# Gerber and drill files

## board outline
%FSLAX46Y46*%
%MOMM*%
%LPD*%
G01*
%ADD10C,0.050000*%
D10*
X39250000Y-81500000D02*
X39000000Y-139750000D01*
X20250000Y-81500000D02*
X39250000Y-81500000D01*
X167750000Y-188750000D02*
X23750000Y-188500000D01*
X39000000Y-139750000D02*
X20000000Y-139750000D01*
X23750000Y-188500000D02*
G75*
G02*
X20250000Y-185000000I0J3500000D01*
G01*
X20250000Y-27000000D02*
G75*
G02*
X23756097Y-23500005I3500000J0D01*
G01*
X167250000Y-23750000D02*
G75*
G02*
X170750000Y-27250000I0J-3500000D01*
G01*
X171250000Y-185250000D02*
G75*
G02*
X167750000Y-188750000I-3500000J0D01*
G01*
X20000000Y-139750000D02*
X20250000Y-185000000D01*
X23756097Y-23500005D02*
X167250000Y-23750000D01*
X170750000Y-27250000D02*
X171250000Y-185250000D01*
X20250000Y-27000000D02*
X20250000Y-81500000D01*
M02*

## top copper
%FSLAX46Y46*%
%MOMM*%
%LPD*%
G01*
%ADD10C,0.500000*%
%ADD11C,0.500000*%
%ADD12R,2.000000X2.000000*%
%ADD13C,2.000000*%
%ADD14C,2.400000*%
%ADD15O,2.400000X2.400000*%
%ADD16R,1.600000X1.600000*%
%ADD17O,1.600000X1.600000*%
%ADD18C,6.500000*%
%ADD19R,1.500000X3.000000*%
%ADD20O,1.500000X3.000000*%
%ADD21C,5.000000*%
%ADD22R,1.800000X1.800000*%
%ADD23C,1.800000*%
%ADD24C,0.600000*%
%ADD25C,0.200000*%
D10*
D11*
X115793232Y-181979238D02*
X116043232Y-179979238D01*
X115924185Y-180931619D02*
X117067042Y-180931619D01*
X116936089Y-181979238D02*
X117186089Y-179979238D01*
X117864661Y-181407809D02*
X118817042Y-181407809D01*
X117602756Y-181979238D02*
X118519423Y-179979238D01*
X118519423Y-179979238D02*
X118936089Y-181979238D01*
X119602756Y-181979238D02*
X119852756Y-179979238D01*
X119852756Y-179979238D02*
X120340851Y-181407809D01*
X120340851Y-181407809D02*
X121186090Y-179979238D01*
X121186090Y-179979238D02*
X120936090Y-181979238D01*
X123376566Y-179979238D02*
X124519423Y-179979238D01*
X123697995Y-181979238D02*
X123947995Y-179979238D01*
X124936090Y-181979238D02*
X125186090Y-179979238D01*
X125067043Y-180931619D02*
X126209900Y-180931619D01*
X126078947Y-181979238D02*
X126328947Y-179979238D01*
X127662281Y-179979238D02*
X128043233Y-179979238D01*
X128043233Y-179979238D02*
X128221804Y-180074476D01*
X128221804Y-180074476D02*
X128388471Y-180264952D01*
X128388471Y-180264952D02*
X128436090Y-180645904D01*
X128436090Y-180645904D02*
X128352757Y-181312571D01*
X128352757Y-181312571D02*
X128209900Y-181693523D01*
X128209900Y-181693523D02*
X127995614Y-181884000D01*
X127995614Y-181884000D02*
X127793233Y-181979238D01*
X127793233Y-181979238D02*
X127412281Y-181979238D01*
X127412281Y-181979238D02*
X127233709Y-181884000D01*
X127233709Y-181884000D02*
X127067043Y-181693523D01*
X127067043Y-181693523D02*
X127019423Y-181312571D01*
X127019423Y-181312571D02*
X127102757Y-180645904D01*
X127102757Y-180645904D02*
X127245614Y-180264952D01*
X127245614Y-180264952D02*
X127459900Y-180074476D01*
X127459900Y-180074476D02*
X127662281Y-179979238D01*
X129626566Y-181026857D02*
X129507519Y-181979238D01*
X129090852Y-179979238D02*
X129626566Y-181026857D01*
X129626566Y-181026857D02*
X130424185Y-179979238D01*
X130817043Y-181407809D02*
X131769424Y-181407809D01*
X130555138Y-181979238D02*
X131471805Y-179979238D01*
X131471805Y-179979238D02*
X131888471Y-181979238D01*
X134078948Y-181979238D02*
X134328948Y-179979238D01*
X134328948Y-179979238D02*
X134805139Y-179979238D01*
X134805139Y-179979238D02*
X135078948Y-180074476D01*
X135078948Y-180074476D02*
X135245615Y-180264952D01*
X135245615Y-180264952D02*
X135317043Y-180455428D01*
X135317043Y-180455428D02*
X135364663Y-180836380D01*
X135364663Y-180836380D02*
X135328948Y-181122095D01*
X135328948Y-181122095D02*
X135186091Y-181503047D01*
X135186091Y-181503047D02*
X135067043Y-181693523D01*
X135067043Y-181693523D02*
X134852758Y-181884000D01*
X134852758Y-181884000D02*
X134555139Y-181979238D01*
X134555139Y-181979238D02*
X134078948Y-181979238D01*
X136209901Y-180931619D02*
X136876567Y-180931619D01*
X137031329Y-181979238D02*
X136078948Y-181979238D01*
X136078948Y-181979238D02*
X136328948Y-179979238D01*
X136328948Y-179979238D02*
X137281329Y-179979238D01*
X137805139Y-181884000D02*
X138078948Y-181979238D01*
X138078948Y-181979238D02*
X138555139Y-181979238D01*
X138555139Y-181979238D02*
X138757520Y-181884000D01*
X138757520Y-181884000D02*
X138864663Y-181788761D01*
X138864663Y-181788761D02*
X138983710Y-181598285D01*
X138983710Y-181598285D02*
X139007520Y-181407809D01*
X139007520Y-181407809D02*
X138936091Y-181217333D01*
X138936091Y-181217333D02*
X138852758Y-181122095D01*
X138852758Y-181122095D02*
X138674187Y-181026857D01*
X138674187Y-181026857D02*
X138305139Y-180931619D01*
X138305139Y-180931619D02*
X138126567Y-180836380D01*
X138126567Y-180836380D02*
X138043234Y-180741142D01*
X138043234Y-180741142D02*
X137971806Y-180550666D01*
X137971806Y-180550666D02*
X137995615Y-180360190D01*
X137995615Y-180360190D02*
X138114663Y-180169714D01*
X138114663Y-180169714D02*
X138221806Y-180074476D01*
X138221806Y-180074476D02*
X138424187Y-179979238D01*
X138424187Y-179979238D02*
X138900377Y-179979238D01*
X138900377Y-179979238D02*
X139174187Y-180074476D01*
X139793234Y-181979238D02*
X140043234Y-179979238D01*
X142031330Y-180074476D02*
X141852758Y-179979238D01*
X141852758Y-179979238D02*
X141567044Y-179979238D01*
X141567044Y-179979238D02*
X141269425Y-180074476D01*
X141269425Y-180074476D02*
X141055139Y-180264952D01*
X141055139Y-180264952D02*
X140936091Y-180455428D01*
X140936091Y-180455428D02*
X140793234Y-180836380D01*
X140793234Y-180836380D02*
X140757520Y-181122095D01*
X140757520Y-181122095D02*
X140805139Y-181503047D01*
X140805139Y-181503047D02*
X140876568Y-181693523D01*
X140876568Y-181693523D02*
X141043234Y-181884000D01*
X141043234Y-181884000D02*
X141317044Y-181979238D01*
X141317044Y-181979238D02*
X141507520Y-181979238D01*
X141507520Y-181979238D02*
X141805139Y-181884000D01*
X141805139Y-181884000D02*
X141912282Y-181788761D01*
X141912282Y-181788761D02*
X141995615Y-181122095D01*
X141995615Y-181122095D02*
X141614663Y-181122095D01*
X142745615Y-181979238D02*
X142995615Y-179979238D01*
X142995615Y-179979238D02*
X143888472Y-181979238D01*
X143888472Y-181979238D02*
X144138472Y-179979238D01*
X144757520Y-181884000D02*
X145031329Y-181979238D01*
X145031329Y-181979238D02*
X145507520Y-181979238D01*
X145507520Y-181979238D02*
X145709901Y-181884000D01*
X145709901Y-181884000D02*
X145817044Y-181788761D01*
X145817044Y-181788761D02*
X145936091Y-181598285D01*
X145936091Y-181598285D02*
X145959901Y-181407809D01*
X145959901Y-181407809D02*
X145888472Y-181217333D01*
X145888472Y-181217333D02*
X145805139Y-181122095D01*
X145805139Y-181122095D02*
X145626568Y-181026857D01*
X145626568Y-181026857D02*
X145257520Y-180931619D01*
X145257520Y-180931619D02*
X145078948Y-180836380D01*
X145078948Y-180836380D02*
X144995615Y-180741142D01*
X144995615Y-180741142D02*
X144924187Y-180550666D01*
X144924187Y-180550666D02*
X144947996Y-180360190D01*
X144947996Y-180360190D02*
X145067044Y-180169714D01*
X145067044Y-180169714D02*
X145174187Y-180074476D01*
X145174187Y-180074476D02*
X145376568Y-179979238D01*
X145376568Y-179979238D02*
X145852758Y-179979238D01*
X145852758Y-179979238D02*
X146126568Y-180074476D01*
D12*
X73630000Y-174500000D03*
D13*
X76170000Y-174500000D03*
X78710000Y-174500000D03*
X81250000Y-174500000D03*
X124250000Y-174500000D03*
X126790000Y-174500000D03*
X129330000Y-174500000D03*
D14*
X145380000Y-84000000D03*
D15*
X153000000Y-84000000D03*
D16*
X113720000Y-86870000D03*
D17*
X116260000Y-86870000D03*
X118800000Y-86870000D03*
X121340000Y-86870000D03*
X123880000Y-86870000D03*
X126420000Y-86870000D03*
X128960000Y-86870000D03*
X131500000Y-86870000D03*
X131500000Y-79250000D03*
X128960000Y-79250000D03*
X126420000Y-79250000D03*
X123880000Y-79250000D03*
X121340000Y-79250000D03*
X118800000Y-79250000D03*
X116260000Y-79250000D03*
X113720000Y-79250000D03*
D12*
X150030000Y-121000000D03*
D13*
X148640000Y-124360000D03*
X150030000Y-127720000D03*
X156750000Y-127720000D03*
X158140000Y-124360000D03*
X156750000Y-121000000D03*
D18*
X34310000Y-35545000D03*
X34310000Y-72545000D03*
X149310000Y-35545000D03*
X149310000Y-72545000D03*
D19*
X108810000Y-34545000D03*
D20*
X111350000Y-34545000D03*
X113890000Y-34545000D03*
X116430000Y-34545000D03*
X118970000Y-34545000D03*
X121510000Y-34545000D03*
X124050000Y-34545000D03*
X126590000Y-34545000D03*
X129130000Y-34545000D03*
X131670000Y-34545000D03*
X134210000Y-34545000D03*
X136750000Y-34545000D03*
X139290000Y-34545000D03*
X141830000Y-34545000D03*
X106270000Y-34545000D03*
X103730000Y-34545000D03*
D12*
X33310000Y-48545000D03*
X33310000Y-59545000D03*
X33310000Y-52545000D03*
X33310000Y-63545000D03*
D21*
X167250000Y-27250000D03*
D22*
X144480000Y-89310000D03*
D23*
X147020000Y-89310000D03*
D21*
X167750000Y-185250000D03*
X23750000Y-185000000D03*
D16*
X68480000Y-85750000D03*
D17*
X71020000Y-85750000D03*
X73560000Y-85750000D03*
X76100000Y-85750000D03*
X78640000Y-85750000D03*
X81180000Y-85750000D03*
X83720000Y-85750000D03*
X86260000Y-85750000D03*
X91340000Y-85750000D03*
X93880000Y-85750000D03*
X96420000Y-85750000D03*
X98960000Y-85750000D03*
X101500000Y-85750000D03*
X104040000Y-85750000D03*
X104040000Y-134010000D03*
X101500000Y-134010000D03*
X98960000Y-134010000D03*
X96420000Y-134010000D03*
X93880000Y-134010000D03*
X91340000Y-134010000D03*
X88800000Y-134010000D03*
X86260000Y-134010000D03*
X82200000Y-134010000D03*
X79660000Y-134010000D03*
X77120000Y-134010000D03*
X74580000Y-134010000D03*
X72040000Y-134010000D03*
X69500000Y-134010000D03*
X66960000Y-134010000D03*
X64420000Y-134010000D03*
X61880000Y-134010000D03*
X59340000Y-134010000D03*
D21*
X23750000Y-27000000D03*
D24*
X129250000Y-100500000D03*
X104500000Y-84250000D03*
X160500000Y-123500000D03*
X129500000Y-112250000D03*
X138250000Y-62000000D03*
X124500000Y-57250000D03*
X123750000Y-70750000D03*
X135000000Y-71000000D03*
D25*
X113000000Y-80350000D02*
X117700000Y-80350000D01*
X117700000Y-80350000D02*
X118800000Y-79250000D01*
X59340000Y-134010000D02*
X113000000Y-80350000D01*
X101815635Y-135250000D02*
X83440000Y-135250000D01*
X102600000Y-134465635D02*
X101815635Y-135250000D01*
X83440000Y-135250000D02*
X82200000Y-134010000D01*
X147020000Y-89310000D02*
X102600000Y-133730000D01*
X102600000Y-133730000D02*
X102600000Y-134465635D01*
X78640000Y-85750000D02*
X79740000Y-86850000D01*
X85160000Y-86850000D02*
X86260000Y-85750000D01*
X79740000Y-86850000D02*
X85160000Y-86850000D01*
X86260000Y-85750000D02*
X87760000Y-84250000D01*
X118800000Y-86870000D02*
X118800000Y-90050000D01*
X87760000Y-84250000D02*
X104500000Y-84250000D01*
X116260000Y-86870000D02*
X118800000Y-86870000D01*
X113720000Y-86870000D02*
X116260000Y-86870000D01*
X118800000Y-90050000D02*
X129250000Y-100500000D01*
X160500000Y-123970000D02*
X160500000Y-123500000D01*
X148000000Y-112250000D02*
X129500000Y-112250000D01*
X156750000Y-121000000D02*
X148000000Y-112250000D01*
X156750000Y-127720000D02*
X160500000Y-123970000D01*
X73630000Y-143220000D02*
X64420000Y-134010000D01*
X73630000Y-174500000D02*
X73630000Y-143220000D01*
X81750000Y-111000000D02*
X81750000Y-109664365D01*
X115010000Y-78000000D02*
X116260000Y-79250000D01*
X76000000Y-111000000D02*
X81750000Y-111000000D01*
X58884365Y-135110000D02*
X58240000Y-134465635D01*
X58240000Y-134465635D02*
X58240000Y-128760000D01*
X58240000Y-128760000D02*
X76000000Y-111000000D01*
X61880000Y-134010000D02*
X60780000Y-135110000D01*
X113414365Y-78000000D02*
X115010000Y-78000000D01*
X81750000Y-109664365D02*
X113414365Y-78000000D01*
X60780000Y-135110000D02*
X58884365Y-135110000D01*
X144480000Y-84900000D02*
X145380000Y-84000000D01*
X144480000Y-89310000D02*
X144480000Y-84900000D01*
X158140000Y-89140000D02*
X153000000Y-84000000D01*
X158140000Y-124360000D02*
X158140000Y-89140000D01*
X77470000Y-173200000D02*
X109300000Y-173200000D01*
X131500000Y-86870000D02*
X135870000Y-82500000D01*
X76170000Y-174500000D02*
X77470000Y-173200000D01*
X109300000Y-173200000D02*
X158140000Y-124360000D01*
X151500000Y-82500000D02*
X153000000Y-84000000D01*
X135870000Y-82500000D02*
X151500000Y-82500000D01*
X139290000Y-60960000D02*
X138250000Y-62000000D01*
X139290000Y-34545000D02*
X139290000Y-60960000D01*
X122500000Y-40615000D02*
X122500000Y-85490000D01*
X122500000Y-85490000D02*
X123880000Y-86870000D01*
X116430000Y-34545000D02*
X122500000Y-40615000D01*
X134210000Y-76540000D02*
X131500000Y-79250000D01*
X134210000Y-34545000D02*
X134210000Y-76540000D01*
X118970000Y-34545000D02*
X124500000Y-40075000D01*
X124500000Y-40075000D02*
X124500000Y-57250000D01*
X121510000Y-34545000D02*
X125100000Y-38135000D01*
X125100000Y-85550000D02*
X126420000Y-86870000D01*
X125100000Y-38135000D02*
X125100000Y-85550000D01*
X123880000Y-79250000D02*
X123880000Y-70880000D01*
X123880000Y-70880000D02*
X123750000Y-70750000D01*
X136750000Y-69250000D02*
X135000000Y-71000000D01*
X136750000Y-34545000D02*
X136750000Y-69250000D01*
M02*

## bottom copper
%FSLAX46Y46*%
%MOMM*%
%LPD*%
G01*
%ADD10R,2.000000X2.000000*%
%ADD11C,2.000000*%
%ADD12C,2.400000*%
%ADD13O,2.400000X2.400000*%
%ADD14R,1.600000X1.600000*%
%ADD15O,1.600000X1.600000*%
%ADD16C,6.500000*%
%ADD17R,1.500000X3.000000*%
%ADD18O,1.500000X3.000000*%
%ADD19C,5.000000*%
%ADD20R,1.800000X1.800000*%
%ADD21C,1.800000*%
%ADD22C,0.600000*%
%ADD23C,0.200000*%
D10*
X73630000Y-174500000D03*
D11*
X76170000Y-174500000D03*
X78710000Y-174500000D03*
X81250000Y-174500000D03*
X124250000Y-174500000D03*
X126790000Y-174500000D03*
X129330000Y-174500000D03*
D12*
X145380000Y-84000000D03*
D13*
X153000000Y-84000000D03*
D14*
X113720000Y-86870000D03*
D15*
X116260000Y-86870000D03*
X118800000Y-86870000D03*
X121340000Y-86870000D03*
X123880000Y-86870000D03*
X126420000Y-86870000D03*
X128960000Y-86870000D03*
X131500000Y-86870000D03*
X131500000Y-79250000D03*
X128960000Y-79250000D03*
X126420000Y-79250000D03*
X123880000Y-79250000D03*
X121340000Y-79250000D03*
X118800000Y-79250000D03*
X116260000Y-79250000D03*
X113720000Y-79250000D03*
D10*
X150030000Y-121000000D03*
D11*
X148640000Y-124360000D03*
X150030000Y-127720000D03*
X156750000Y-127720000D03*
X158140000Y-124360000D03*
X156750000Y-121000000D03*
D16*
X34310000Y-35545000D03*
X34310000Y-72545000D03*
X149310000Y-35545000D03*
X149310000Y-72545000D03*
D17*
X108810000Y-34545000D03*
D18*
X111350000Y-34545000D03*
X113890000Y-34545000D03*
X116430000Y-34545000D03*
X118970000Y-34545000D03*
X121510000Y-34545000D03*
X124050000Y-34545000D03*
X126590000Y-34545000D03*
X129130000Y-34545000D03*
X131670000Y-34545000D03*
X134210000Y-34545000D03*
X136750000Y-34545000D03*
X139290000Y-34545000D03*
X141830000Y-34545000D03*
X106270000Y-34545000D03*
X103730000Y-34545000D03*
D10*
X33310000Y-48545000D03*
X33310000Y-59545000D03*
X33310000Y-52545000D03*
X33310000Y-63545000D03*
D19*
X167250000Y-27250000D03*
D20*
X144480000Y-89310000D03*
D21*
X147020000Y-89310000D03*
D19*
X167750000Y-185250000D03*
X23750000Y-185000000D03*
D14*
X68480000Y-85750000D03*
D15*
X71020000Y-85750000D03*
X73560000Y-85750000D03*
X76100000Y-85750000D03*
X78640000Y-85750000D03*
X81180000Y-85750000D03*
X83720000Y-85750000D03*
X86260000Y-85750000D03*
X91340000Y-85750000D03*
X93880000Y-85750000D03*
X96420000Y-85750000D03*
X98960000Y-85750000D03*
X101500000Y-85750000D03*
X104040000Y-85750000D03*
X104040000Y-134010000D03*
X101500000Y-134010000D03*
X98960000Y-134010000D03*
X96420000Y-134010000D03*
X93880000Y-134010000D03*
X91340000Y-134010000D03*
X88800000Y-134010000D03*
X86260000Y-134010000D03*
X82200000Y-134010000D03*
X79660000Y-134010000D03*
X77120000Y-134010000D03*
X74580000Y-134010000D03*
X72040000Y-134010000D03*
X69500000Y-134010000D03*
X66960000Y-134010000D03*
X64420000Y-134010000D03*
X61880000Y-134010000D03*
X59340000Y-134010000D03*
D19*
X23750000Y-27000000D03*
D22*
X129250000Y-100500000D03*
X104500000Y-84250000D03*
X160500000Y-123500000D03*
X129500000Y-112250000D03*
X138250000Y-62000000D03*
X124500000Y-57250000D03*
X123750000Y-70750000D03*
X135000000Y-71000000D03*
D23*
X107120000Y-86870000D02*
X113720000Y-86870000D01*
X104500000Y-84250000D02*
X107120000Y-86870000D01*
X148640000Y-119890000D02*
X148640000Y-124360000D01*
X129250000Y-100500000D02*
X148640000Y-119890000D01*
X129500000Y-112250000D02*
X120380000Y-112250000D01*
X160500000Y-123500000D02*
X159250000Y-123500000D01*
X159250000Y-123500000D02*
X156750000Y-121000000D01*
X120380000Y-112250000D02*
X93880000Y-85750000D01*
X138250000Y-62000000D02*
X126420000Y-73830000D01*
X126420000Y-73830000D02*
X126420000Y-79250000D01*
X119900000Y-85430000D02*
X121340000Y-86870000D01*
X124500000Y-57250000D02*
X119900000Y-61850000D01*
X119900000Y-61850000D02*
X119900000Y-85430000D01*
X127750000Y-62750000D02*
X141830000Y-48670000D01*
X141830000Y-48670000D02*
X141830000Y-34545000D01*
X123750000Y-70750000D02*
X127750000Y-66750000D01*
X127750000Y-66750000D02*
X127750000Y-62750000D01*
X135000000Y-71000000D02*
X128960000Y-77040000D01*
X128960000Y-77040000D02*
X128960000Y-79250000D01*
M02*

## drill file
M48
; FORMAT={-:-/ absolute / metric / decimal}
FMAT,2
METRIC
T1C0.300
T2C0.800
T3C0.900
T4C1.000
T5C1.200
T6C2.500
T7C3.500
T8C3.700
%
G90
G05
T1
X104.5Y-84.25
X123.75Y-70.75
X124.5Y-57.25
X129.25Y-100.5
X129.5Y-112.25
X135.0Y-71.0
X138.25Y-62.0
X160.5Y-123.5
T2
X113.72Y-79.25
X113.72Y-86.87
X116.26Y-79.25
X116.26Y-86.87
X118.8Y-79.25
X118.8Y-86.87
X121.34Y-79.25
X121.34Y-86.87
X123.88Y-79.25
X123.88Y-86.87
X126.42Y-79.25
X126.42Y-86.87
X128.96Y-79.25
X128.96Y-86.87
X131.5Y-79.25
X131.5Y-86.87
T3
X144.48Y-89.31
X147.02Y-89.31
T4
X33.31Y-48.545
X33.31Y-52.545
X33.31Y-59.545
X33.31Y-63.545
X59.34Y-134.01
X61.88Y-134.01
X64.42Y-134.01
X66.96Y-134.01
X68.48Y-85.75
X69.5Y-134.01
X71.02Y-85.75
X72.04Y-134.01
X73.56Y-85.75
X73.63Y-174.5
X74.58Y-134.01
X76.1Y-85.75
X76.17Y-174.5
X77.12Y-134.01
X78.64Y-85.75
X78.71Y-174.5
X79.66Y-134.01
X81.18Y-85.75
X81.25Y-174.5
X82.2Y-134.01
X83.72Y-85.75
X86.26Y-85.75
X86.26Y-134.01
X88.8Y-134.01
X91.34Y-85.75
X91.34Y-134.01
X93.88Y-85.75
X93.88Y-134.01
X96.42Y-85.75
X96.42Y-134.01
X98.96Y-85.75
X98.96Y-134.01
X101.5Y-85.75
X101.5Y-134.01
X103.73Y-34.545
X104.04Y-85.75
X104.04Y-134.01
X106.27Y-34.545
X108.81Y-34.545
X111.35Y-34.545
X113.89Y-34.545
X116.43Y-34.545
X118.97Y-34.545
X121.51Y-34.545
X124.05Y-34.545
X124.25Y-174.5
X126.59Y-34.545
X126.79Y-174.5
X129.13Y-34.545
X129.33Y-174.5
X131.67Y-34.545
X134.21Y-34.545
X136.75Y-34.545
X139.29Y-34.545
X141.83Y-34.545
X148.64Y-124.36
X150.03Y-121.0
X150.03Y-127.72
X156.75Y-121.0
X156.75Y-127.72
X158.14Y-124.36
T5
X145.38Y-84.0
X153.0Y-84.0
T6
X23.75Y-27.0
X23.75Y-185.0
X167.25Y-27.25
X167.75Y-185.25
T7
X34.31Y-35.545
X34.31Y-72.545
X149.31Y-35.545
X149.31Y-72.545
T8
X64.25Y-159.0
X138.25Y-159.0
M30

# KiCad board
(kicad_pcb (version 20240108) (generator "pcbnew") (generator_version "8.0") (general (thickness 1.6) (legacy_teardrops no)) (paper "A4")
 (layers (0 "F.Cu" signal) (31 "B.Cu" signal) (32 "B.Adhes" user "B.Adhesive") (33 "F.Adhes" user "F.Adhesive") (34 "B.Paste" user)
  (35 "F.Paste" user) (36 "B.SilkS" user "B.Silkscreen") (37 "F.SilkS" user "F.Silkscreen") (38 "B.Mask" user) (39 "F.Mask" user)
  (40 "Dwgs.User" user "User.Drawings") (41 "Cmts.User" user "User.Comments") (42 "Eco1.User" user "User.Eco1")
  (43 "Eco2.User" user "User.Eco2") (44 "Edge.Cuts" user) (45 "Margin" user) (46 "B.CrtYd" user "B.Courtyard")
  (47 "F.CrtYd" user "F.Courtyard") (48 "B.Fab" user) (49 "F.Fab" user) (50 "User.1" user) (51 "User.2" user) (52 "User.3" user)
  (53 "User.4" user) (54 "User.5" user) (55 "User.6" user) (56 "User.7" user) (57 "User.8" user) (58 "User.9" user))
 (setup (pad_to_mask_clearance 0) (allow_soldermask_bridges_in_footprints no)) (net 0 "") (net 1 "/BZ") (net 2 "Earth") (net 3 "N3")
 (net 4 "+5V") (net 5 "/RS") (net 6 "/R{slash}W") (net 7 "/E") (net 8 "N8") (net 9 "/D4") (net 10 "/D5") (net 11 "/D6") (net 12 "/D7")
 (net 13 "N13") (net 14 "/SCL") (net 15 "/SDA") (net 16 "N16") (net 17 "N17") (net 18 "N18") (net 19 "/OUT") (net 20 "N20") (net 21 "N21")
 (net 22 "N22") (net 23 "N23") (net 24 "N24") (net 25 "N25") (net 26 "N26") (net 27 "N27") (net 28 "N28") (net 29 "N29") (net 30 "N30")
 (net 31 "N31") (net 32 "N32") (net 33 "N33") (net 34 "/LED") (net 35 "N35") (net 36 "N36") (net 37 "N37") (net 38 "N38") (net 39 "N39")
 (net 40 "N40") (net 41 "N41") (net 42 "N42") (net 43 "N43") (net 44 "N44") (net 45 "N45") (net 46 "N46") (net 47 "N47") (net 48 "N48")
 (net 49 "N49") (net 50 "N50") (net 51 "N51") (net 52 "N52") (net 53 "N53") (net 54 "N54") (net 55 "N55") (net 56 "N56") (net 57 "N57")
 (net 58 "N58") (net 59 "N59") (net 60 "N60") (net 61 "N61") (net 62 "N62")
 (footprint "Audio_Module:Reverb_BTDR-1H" (layer "F.Cu") (at 73.63 174.5)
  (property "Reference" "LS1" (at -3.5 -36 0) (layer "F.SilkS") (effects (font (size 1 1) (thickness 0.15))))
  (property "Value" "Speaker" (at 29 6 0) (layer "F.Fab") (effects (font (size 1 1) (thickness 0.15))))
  (pad "" np_thru_hole circle (at -9.38 -15.5) (size 3.7 3.7) (drill 3.7) (layers "*.Cu" "*.Mask"))
  (pad "" np_thru_hole circle (at 64.62 -15.5) (size 3.7 3.7) (drill 3.7) (layers "*.Cu" "*.Mask"))
  (pad "1" thru_hole rect (at 0 0) (size 2 2) (drill 1) (layers "*.Cu" "*.Mask") (remove_unused_layers no) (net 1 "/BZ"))
  (pad "2" thru_hole circle (at 2.54 0) (size 2 2) (drill 1) (layers "*.Cu" "*.Mask") (remove_unused_layers no) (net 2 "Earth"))
  (pad "3" thru_hole circle (at 5.08 0) (size 2 2) (drill 1) (layers "*.Cu" "*.Mask") (remove_unused_layers no))
  (pad "4" thru_hole circle (at 7.62 0) (size 2 2) (drill 1) (layers "*.Cu" "*.Mask") (remove_unused_layers no))
  (pad "5" thru_hole circle (at 50.62 0) (size 2 2) (drill 1) (layers "*.Cu" "*.Mask") (remove_unused_layers no))
  (pad "6" thru_hole circle (at 53.16 0) (size 2 2) (drill 1) (layers "*.Cu" "*.Mask") (remove_unused_layers no))
  (pad "7" thru_hole circle (at 55.7 0) (size 2 2) (drill 1) (layers "*.Cu" "*.Mask") (remove_unused_layers no)))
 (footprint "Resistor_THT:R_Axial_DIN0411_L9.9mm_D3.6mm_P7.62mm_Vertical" (layer "F.Cu") (at 145.38 84)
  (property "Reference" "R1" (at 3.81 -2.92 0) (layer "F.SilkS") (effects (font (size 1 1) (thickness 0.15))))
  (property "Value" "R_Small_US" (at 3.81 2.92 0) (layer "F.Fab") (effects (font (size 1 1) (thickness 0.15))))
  (pad "1" thru_hole circle (at 0 0) (size 2.4 2.4) (drill 1.2) (layers "*.Cu" "*.Mask") (remove_unused_layers no) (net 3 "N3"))
  (pad "2" thru_hole oval (at 7.62 0) (size 2.4 2.4) (drill 1.2) (layers "*.Cu" "*.Mask") (remove_unused_layers no) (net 2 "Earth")))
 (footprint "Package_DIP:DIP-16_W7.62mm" (layer "F.Cu") (at 113.72 86.87 90)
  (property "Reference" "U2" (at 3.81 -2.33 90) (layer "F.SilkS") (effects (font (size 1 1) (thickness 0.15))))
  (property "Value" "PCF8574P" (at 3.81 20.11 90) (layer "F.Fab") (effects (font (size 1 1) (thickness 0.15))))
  (pad "1" thru_hole rect (at 0 0 90) (size 1.6 1.6) (drill 0.8) (layers "*.Cu" "*.Mask") (remove_unused_layers no) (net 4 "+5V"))
  (pad "2" thru_hole oval (at 0 2.54 90) (size 1.6 1.6) (drill 0.8) (layers "*.Cu" "*.Mask") (remove_unused_layers no) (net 4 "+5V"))
  (pad "3" thru_hole oval (at 0 5.08 90) (size 1.6 1.6) (drill 0.8) (layers "*.Cu" "*.Mask") (remove_unused_layers no) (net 4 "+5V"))
  (pad "4" thru_hole oval (at 0 7.62 90) (size 1.6 1.6) (drill 0.8) (layers "*.Cu" "*.Mask") (remove_unused_layers no) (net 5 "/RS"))
  (pad "5" thru_hole oval (at 0 10.16 90) (size 1.6 1.6) (drill 0.8) (layers "*.Cu" "*.Mask") (remove_unused_layers no) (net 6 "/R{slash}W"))
  (pad "6" thru_hole oval (at 0 12.7 90) (size 1.6 1.6) (drill 0.8) (layers "*.Cu" "*.Mask") (remove_unused_layers no) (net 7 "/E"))
  (pad "7" thru_hole oval (at 0 15.24 90) (size 1.6 1.6) (drill 0.8) (layers "*.Cu" "*.Mask") (remove_unused_layers no) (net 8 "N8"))
  (pad "8" thru_hole oval (at 0 17.78 90) (size 1.6 1.6) (drill 0.8) (layers "*.Cu" "*.Mask") (remove_unused_layers no) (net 2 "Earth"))
  (pad "9" thru_hole oval (at 7.62 17.78 90) (size 1.6 1.6) (drill 0.8) (layers "*.Cu" "*.Mask") (remove_unused_layers no) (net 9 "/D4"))
  (pad "10" thru_hole oval (at 7.62 15.24 90) (size 1.6 1.6) (drill 0.8) (layers "*.Cu" "*.Mask") (remove_unused_layers no) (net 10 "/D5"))
  (pad "11" thru_hole oval (at 7.62 12.7 90) (size 1.6 1.6) (drill 0.8) (layers "*.Cu" "*.Mask") (remove_unused_layers no) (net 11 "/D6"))
  (pad "12" thru_hole oval (at 7.62 10.16 90) (size 1.6 1.6) (drill 0.8) (layers "*.Cu" "*.Mask") (remove_unused_layers no) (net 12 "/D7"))
  (pad "13" thru_hole oval (at 7.62 7.62 90) (size 1.6 1.6) (drill 0.8) (layers "*.Cu" "*.Mask") (remove_unused_layers no) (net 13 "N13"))
  (pad "14" thru_hole oval (at 7.62 5.08 90) (size 1.6 1.6) (drill 0.8) (layers "*.Cu" "*.Mask") (remove_unused_layers no) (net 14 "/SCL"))
  (pad "15" thru_hole oval (at 7.62 2.54 90) (size 1.6 1.6) (drill 0.8) (layers "*.Cu" "*.Mask") (remove_unused_layers no) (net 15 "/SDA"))
  (pad "16" thru_hole oval (at 7.62 0 90) (size 1.6 1.6) (drill 0.8) (layers "*.Cu" "*.Mask") (remove_unused_layers no) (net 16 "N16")))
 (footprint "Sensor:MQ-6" (layer "F.Cu") (at 150.03 121)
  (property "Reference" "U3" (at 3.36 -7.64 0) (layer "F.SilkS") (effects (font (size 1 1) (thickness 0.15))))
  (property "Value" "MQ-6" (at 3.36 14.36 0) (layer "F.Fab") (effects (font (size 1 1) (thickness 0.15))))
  (pad "1" thru_hole rect (at 0 0) (size 2 2) (drill 1) (layers "*.Cu" "*.Mask") (remove_unused_layers no) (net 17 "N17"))
  (pad "2" thru_hole circle (at -1.39 3.36) (size 2 2) (drill 1) (layers "*.Cu" "*.Mask") (remove_unused_layers no) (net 4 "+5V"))
  (pad "3" thru_hole circle (at 0 6.72 90) (size 2 2) (drill 1) (layers "*.Cu" "*.Mask") (remove_unused_layers no) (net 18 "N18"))
  (pad "4" thru_hole circle (at 6.72 6.72 180) (size 2 2) (drill 1) (layers "*.Cu" "*.Mask") (remove_unused_layers no) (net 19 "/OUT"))
  (pad "5" thru_hole circle (at 8.11 3.36) (size 2 2) (drill 1) (layers "*.Cu" "*.Mask") (remove_unused_layers no) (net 2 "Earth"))
  (pad "6" thru_hole circle (at 6.72 0 270) (size 2 2) (drill 1) (layers "*.Cu" "*.Mask") (remove_unused_layers no) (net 19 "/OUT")))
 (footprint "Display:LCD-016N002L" (layer "F.Cu") (at 108.81 34.545)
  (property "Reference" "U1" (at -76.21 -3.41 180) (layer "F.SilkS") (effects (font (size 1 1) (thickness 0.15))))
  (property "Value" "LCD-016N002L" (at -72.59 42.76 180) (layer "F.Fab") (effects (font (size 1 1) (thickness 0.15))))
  (pad "" thru_hole circle (at -74.5 1 180) (size 6.5 6.5) (drill 3.5) (layers "*.Cu" "*.Mask") (remove_unused_layers no))
  (pad "" thru_hole circle (at -74.5 38 180) (size 6.5 6.5) (drill 3.5) (layers "*.Cu" "*.Mask") (remove_unused_layers no))
  (pad "" thru_hole circle (at 40.5 1 180) (size 6.5 6.5) (drill 3.5) (layers "*.Cu" "*.Mask") (remove_unused_layers no))
  (pad "" thru_hole circle (at 40.5 38 180) (size 6.5 6.5) (drill 3.5) (layers "*.Cu" "*.Mask") (remove_unused_layers no))
  (pad "1" thru_hole rect (at 0 0 180) (size 1.5 3) (drill 1) (layers "*.Cu" "*.Mask") (remove_unused_layers no) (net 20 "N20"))
  (pad "2" thru_hole oval (at 2.54 0 180) (size 1.5 3) (drill 1) (layers "*.Cu" "*.Mask") (remove_unused_layers no) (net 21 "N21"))
  (pad "3" thru_hole oval (at 5.08 0 180) (size 1.5 3) (drill 1) (layers "*.Cu" "*.Mask") (remove_unused_layers no) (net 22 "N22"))
  (pad "4" thru_hole oval (at 7.62 0 180) (size 1.5 3) (drill 1) (layers "*.Cu" "*.Mask") (remove_unused_layers no) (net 6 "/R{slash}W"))
  (pad "5" thru_hole oval (at 10.16 0 180) (size 1.5 3) (drill 1) (layers "*.Cu" "*.Mask") (remove_unused_layers no) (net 5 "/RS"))
  (pad "6" thru_hole oval (at 12.7 0 180) (size 1.5 3) (drill 1) (layers "*.Cu" "*.Mask") (remove_unused_layers no) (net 7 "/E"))
  (pad "7" thru_hole oval (at 15.24 0 180) (size 1.5 3) (drill 1) (layers "*.Cu" "*.Mask") (remove_unused_layers no) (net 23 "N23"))
  (pad "8" thru_hole oval (at 17.78 0 180) (size 1.5 3) (drill 1) (layers "*.Cu" "*.Mask") (remove_unused_layers no) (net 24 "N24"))
  (pad "9" thru_hole oval (at 20.32 0 180) (size 1.5 3) (drill 1) (layers "*.Cu" "*.Mask") (remove_unused_layers no) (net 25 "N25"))
  (pad "10" thru_hole oval (at 22.86 0 180) (size 1.5 3) (drill 1) (layers "*.Cu" "*.Mask") (remove_unused_layers no) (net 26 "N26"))
  (pad "11" thru_hole oval (at 25.4 0 180) (size 1.5 3) (drill 1) (layers "*.Cu" "*.Mask") (remove_unused_layers no) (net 9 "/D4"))
  (pad "12" thru_hole oval (at 27.94 0 180) (size 1.5 3) (drill 1) (layers "*.Cu" "*.Mask") (remove_unused_layers no) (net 10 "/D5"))
  (pad "13" thru_hole oval (at 30.48 0 180) (size 1.5 3) (drill 1) (layers "*.Cu" "*.Mask") (remove_unused_layers no) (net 11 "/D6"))
  (pad "14" thru_hole oval (at 33.02 0 180) (size 1.5 3) (drill 1) (layers "*.Cu" "*.Mask") (remove_unused_layers no) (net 12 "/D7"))
  (pad "15" thru_hole oval (at -2.54 0 180) (size 1.5 3) (drill 1) (layers "*.Cu" "*.Mask") (remove_unused_layers no) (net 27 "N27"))
  (pad "16" thru_hole oval (at -5.08 0 180) (size 1.5 3) (drill 1) (layers "*.Cu" "*.Mask") (remove_unused_layers no) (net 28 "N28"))
  (pad "A1" thru_hole rect (at -75.5 14 180) (size 2 2) (drill 1) (layers "*.Cu" "*.Mask") (remove_unused_layers no) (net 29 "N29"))
  (pad "A2" thru_hole rect (at -75.5 25 180) (size 2 2) (drill 1) (layers "*.Cu" "*.Mask") (remove_unused_layers no) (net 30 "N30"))
  (pad "K1" thru_hole rect (at -75.5 18 180) (size 2 2) (drill 1) (layers "*.Cu" "*.Mask") (remove_unused_layers no) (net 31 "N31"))
  (pad "K2" thru_hole rect (at -75.5 29 180) (size 2 2) (drill 1) (layers "*.Cu" "*.Mask") (remove_unused_layers no) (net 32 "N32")))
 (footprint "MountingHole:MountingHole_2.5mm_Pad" (layer "F.Cu") (at 167.25 27.25)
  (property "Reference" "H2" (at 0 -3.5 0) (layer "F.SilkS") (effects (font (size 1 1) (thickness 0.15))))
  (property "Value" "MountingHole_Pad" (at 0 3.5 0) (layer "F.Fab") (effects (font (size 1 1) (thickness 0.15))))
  (pad "1" thru_hole circle (at 0 0) (size 5 5) (drill 2.5) (layers "*.Cu" "*.Mask") (remove_unused_layers no) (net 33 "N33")))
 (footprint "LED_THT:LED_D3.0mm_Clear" (layer "F.Cu") (at 144.48 89.31)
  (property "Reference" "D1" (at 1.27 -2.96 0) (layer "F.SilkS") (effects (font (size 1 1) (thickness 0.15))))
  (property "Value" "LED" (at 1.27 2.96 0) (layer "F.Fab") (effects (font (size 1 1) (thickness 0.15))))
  (pad "1" thru_hole rect (at 0 0) (size 1.8 1.8) (drill 0.9) (layers "*.Cu" "*.Mask") (remove_unused_layers no) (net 3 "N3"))
  (pad "2" thru_hole circle (at 2.54 0) (size 1.8 1.8) (drill 0.9) (layers "*.Cu" "*.Mask") (remove_unused_layers no) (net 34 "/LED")))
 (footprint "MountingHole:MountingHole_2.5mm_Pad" (layer "F.Cu") (at 167.75 185.25)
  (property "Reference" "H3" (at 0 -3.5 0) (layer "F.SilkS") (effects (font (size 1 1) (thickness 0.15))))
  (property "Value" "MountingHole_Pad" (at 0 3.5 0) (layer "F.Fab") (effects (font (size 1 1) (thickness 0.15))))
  (pad "1" thru_hole circle (at 0 0) (size 5 5) (drill 2.5) (layers "*.Cu" "*.Mask") (remove_unused_layers no) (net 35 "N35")))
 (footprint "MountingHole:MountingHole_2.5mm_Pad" (layer "F.Cu") (at 23.75 185)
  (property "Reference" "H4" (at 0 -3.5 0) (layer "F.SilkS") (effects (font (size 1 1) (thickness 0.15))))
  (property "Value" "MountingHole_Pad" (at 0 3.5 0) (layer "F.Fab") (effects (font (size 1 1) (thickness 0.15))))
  (pad "1" thru_hole circle (at 0 0) (size 5 5) (drill 2.5) (layers "*.Cu" "*.Mask") (remove_unused_layers no) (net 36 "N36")))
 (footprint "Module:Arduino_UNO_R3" (layer "F.Cu") (at 68.48 85.75)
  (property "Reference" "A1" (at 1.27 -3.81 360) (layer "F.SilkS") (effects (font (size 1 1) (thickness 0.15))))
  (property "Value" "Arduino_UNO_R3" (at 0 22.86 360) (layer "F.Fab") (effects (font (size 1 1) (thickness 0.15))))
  (pad "1" thru_hole rect (at 0 0 90) (size 1.6 1.6) (drill 1) (layers "*.Cu" "*.Mask") (remove_unused_layers no) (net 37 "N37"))
  (pad "2" thru_hole oval (at 2.54 0 90) (size 1.6 1.6) (drill 1) (layers "*.Cu" "*.Mask") (remove_unused_layers no) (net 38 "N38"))
  (pad "3" thru_hole oval (at 5.08 0 90) (size 1.6 1.6) (drill 1) (layers "*.Cu" "*.Mask") (remove_unused_layers no) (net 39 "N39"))
  (pad "4" thru_hole oval (at 7.62 0 90) (size 1.6 1.6) (drill 1) (layers "*.Cu" "*.Mask") (remove_unused_layers no) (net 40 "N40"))
  (pad "5" thru_hole oval (at 10.16 0 90) (size 1.6 1.6) (drill 1) (layers "*.Cu" "*.Mask") (remove_unused_layers no) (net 4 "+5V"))
  (pad "6" thru_hole oval (at 12.7 0 90) (size 1.6 1.6) (drill 1) (layers "*.Cu" "*.Mask") (remove_unused_layers no) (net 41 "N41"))
  (pad "7" thru_hole oval (at 15.24 0 90) (size 1.6 1.6) (drill 1) (layers "*.Cu" "*.Mask") (remove_unused_layers no) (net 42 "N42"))
  (pad "8" thru_hole oval (at 17.78 0 90) (size 1.6 1.6) (drill 1) (layers "*.Cu" "*.Mask") (remove_unused_layers no) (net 4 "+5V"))
  (pad "9" thru_hole oval (at 22.86 0 90) (size 1.6 1.6) (drill 1) (layers "*.Cu" "*.Mask") (remove_unused_layers no) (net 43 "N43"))
  (pad "10" thru_hole oval (at 25.4 0 90) (size 1.6 1.6) (drill 1) (layers "*.Cu" "*.Mask") (remove_unused_layers no) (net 19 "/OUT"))
  (pad "11" thru_hole oval (at 27.94 0 90) (size 1.6 1.6) (drill 1) (layers "*.Cu" "*.Mask") (remove_unused_layers no) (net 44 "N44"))
  (pad "12" thru_hole oval (at 30.48 0 90) (size 1.6 1.6) (drill 1) (layers "*.Cu" "*.Mask") (remove_unused_layers no) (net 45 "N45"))
  (pad "13" thru_hole oval (at 33.02 0 90) (size 1.6 1.6) (drill 1) (layers "*.Cu" "*.Mask") (remove_unused_layers no) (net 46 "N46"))
  (pad "14" thru_hole oval (at 35.56 0 90) (size 1.6 1.6) (drill 1) (layers "*.Cu" "*.Mask") (remove_unused_layers no) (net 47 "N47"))
  (pad "15" thru_hole oval (at 35.56 48.26 90) (size 1.6 1.6) (drill 1) (layers "*.Cu" "*.Mask") (remove_unused_layers no) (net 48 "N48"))
  (pad "16" thru_hole oval (at 33.02 48.26 90) (size 1.6 1.6) (drill 1) (layers "*.Cu" "*.Mask") (remove_unused_layers no) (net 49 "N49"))
  (pad "17" thru_hole oval (at 30.48 48.26 90) (size 1.6 1.6) (drill 1) (layers "*.Cu" "*.Mask") (remove_unused_layers no) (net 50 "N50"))
  (pad "18" thru_hole oval (at 27.94 48.26 90) (size 1.6 1.6) (drill 1) (layers "*.Cu" "*.Mask") (remove_unused_layers no) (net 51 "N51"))
  (pad "19" thru_hole oval (at 25.4 48.26 90) (size 1.6 1.6) (drill 1) (layers "*.Cu" "*.Mask") (remove_unused_layers no) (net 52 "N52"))
  (pad "20" thru_hole oval (at 22.86 48.26 90) (size 1.6 1.6) (drill 1) (layers "*.Cu" "*.Mask") (remove_unused_layers no) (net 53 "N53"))
  (pad "21" thru_hole oval (at 20.32 48.26 90) (size 1.6 1.6) (drill 1) (layers "*.Cu" "*.Mask") (remove_unused_layers no) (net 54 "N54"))
  (pad "22" thru_hole oval (at 17.78 48.26 90) (size 1.6 1.6) (drill 1) (layers "*.Cu" "*.Mask") (remove_unused_layers no) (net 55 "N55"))
  (pad "23" thru_hole oval (at 13.72 48.26 90) (size 1.6 1.6) (drill 1) (layers "*.Cu" "*.Mask") (remove_unused_layers no) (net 34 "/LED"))
  (pad "24" thru_hole oval (at 11.18 48.26 90) (size 1.6 1.6) (drill 1) (layers "*.Cu" "*.Mask") (remove_unused_layers no) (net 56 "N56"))
  (pad "25" thru_hole oval (at 8.64 48.26 90) (size 1.6 1.6) (drill 1) (layers "*.Cu" "*.Mask") (remove_unused_layers no) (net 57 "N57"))
  (pad "26" thru_hole oval (at 6.1 48.26 90) (size 1.6 1.6) (drill 1) (layers "*.Cu" "*.Mask") (remove_unused_layers no) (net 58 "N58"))
  (pad "27" thru_hole oval (at 3.56 48.26 90) (size 1.6 1.6) (drill 1) (layers "*.Cu" "*.Mask") (remove_unused_layers no) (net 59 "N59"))
  (pad "28" thru_hole oval (at 1.02 48.26 90) (size 1.6 1.6) (drill 1) (layers "*.Cu" "*.Mask") (remove_unused_layers no) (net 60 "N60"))
  (pad "29" thru_hole oval (at -1.52 48.26 90) (size 1.6 1.6) (drill 1) (layers "*.Cu" "*.Mask") (remove_unused_layers no) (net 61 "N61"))
  (pad "30" thru_hole oval (at -4.06 48.26 90) (size 1.6 1.6) (drill 1) (layers "*.Cu" "*.Mask") (remove_unused_layers no) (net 1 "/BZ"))
  (pad "31" thru_hole oval (at -6.6 48.26 90) (size 1.6 1.6) (drill 1) (layers "*.Cu" "*.Mask") (remove_unused_layers no) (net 15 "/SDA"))
  (pad "32" thru_hole oval (at -9.14 48.26 90) (size 1.6 1.6) (drill 1) (layers "*.Cu" "*.Mask") (remove_unused_layers no) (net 14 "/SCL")))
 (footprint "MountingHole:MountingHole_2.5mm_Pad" (layer "F.Cu") (at 23.75 27)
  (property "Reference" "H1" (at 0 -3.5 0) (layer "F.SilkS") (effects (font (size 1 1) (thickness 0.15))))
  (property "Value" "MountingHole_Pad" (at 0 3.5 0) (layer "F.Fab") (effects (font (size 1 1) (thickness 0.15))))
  (pad "1" thru_hole circle (at 0 0) (size 5 5) (drill 2.5) (layers "*.Cu" "*.Mask") (remove_unused_layers no) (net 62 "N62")))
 (gr_line (start 39.25 81.5) (end 39 139.75) (stroke (width 0.05) (type default)) (layer "Edge.Cuts"))
 (gr_line (start 20.25 81.5) (end 39.25 81.5) (stroke (width 0.05) (type default)) (layer "Edge.Cuts"))
 (gr_line (start 167.75 188.75) (end 23.75 188.5) (stroke (width 0.05) (type default)) (layer "Edge.Cuts"))
 (gr_line (start 39 139.75) (end 20 139.75) (stroke (width 0.05) (type default)) (layer "Edge.Cuts"))
 (gr_arc (start 23.75 188.5) (mid 21.275126 187.474874) (end 20.25 185) (stroke (width 0.05) (type default)) (layer "Edge.Cuts"))
 (gr_arc (start 20.25 27) (mid 21.277283 24.522972) (end 23.756097 23.500005) (stroke (width 0.05) (type default)) (layer "Edge.Cuts"))
 (gr_arc (start 167.25 23.75) (mid 169.724874 24.775126) (end 170.75 27.25) (stroke (width 0.05) (type default)) (layer "Edge.Cuts"))
 (gr_arc (start 171.25 185.25) (mid 170.224874 187.724874) (end 167.75 188.75) (stroke (width 0.05) (type default)) (layer "Edge.Cuts"))
 (gr_line (start 20 139.75) (end 20.25 185) (stroke (width 0.05) (type default)) (layer "Edge.Cuts"))
 (gr_line (start 23.756097 23.500005) (end 167.25 23.75) (stroke (width 0.05) (type default)) (layer "Edge.Cuts"))
 (gr_line (start 170.75 27.25) (end 171.25 185.25) (stroke (width 0.05) (type default)) (layer "Edge.Cuts"))
 (gr_line (start 20.25 27) (end 20.25 81.5) (stroke (width 0.05) (type default)) (layer "Edge.Cuts"))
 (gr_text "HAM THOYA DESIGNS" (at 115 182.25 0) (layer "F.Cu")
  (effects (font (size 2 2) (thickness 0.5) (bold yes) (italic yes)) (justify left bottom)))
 (segment (start 113 80.35) (end 117.7 80.35) (width 0.2) (layer "F.Cu") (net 14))
 (segment (start 117.7 80.35) (end 118.8 79.25) (width 0.2) (layer "F.Cu") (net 14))
 (segment (start 59.34 134.01) (end 113 80.35) (width 0.2) (layer "F.Cu") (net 14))
 (segment (start 101.815635 135.25) (end 83.44 135.25) (width 0.2) (layer "F.Cu") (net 34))
 (segment (start 102.6 134.465635) (end 101.815635 135.25) (width 0.2) (layer "F.Cu") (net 34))
 (segment (start 83.44 135.25) (end 82.2 134.01) (width 0.2) (layer "F.Cu") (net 34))
 (segment (start 147.02 89.31) (end 102.6 133.73) (width 0.2) (layer "F.Cu") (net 34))
 (segment (start 102.6 133.73) (end 102.6 134.465635) (width 0.2) (layer "F.Cu") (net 34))
 (segment (start 78.64 85.75) (end 79.74 86.85) (width 0.2) (layer "F.Cu") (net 4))
 (segment (start 85.16 86.85) (end 86.26 85.75) (width 0.2) (layer "F.Cu") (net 4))
 (segment (start 79.74 86.85) (end 85.16 86.85) (width 0.2) (layer "F.Cu") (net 4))
 (segment (start 86.26 85.75) (end 87.76 84.25) (width 0.2) (layer "F.Cu") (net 4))
 (segment (start 118.8 86.87) (end 118.8 90.05) (width 0.2) (layer "F.Cu") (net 4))
 (segment (start 87.76 84.25) (end 104.5 84.25) (width 0.2) (layer "F.Cu") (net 4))
 (segment (start 116.26 86.87) (end 118.8 86.87) (width 0.2) (layer "F.Cu") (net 4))
 (segment (start 113.72 86.87) (end 116.26 86.87) (width 0.2) (layer "F.Cu") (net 4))
 (segment (start 118.8 90.05) (end 129.25 100.5) (width 0.2) (layer "F.Cu") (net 4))
 (via (at 129.25 100.5) (size 0.6) (drill 0.3) (layers "F.Cu" "B.Cu") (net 4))
 (via (at 104.5 84.25) (size 0.6) (drill 0.3) (layers "F.Cu" "B.Cu") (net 4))
 (segment (start 107.12 86.87) (end 113.72 86.87) (width 0.2) (layer "B.Cu") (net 4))
 (segment (start 104.5 84.25) (end 107.12 86.87) (width 0.2) (layer "B.Cu") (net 4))
 (segment (start 148.64 119.89) (end 148.64 124.36) (width 0.2) (layer "B.Cu") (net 4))
 (segment (start 129.25 100.5) (end 148.64 119.89) (width 0.2) (layer "B.Cu") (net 4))
 (segment (start 160.5 123.97) (end 160.5 123.5) (width 0.2) (layer "F.Cu") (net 19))
 (segment (start 148 112.25) (end 129.5 112.25) (width 0.2) (layer "F.Cu") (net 19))
 (segment (start 156.75 121) (end 148 112.25) (width 0.2) (layer "F.Cu") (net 19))
 (segment (start 156.75 127.72) (end 160.5 123.97) (width 0.2) (layer "F.Cu") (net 19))
 (via (at 160.5 123.5) (size 0.6) (drill 0.3) (layers "F.Cu" "B.Cu") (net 19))
 (via (at 129.5 112.25) (size 0.6) (drill 0.3) (layers "F.Cu" "B.Cu") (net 19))
 (segment (start 129.5 112.25) (end 120.38 112.25) (width 0.2) (layer "B.Cu") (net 19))
 (segment (start 160.5 123.5) (end 159.25 123.5) (width 0.2) (layer "B.Cu") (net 19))
 (segment (start 159.25 123.5) (end 156.75 121) (width 0.2) (layer "B.Cu") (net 19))
 (segment (start 120.38 112.25) (end 93.88 85.75) (width 0.2) (layer "B.Cu") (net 19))
 (segment (start 73.63 143.22) (end 64.42 134.01) (width 0.2) (layer "F.Cu") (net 1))
 (segment (start 73.63 174.5) (end 73.63 143.22) (width 0.2) (layer "F.Cu") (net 1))
 (segment (start 81.75 111) (end 81.75 109.664365) (width 0.2) (layer "F.Cu") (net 15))
 (segment (start 115.01 78) (end 116.26 79.25) (width 0.2) (layer "F.Cu") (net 15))
 (segment (start 76 111) (end 81.75 111) (width 0.2) (layer "F.Cu") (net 15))
 (segment (start 58.884365 135.11) (end 58.24 134.465635) (width 0.2) (layer "F.Cu") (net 15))
 (segment (start 58.24 134.465635) (end 58.24 128.76) (width 0.2) (layer "F.Cu") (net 15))
 (segment (start 58.24 128.76) (end 76 111) (width 0.2) (layer "F.Cu") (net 15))
 (segment (start 61.88 134.01) (end 60.78 135.11) (width 0.2) (layer "F.Cu") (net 15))
 (segment (start 113.414365 78) (end 115.01 78) (width 0.2) (layer "F.Cu") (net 15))
 (segment (start 81.75 109.664365) (end 113.414365 78) (width 0.2) (layer "F.Cu") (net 15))
 (segment (start 60.78 135.11) (end 58.884365 135.11) (width 0.2) (layer "F.Cu") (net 15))
 (segment (start 144.48 84.9) (end 145.38 84) (width 0.2) (layer "F.Cu") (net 3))
 (segment (start 144.48 89.31) (end 144.48 84.9) (width 0.2) (layer "F.Cu") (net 3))
 (segment (start 158.14 89.14) (end 153 84) (width 0.2) (layer "F.Cu") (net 2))
 (segment (start 158.14 124.36) (end 158.14 89.14) (width 0.2) (layer "F.Cu") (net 2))
 (segment (start 77.47 173.2) (end 109.3 173.2) (width 0.2) (layer "F.Cu") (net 2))
 (segment (start 131.5 86.87) (end 135.87 82.5) (width 0.2) (layer "F.Cu") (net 2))
 (segment (start 76.17 174.5) (end 77.47 173.2) (width 0.2) (layer "F.Cu") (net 2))
 (segment (start 109.3 173.2) (end 158.14 124.36) (width 0.2) (layer "F.Cu") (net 2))
 (segment (start 151.5 82.5) (end 153 84) (width 0.2) (layer "F.Cu") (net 2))
 (segment (start 135.87 82.5) (end 151.5 82.5) (width 0.2) (layer "F.Cu") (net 2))
 (segment (start 139.29 60.96) (end 138.25 62) (width 0.2) (layer "F.Cu") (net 11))
 (segment (start 139.29 34.545) (end 139.29 60.96) (width 0.2) (layer "F.Cu") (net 11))
 (via (at 138.25 62) (size 0.6) (drill 0.3) (layers "F.Cu" "B.Cu") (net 11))
 (segment (start 138.25 62) (end 126.42 73.83) (width 0.2) (layer "B.Cu") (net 11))
 (segment (start 126.42 73.83) (end 126.42 79.25) (width 0.2) (layer "B.Cu") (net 11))
 (segment (start 122.5 40.615) (end 122.5 85.49) (width 0.2) (layer "F.Cu") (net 6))
 (segment (start 122.5 85.49) (end 123.88 86.87) (width 0.2) (layer "F.Cu") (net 6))
 (segment (start 116.43 34.545) (end 122.5 40.615) (width 0.2) (layer "F.Cu") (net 6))
 (segment (start 134.21 76.54) (end 131.5 79.25) (width 0.2) (layer "F.Cu") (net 9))
 (segment (start 134.21 34.545) (end 134.21 76.54) (width 0.2) (layer "F.Cu") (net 9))
 (segment (start 118.97 34.545) (end 124.5 40.075) (width 0.2) (layer "F.Cu") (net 5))
 (segment (start 124.5 40.075) (end 124.5 57.25) (width 0.2) (layer "F.Cu") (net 5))
 (via (at 124.5 57.25) (size 0.6) (drill 0.3) (layers "F.Cu" "B.Cu") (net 5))
 (segment (start 119.9 85.43) (end 121.34 86.87) (width 0.2) (layer "B.Cu") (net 5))
 (segment (start 124.5 57.25) (end 119.9 61.85) (width 0.2) (layer "B.Cu") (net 5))
 (segment (start 119.9 61.85) (end 119.9 85.43) (width 0.2) (layer "B.Cu") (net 5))
 (segment (start 121.51 34.545) (end 125.1 38.135) (width 0.2) (layer "F.Cu") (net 7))
 (segment (start 125.1 85.55) (end 126.42 86.87) (width 0.2) (layer "F.Cu") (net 7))
 (segment (start 125.1 38.135) (end 125.1 85.55) (width 0.2) (layer "F.Cu") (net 7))
 (segment (start 123.88 79.25) (end 123.88 70.88) (width 0.2) (layer "F.Cu") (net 12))
 (segment (start 123.88 70.88) (end 123.75 70.75) (width 0.2) (layer "F.Cu") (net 12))
 (via (at 123.75 70.75) (size 0.6) (drill 0.3) (layers "F.Cu" "B.Cu") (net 12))
 (segment (start 127.75 62.75) (end 141.83 48.67) (width 0.2) (layer "B.Cu") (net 12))
 (segment (start 141.83 48.67) (end 141.83 34.545) (width 0.2) (layer "B.Cu") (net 12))
 (segment (start 123.75 70.75) (end 127.75 66.75) (width 0.2) (layer "B.Cu") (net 12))
 (segment (start 127.75 66.75) (end 127.75 62.75) (width 0.2) (layer "B.Cu") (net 12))
 (segment (start 136.75 69.25) (end 135 71) (width 0.2) (layer "F.Cu") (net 10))
 (segment (start 136.75 34.545) (end 136.75 69.25) (width 0.2) (layer "F.Cu") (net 10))
 (via (at 135 71) (size 0.6) (drill 0.3) (layers "F.Cu" "B.Cu") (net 10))
 (segment (start 135 71) (end 128.96 77.04) (width 0.2) (layer "B.Cu") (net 10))
 (segment (start 128.96 77.04) (end 128.96 79.25) (width 0.2) (layer "B.Cu") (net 10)))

